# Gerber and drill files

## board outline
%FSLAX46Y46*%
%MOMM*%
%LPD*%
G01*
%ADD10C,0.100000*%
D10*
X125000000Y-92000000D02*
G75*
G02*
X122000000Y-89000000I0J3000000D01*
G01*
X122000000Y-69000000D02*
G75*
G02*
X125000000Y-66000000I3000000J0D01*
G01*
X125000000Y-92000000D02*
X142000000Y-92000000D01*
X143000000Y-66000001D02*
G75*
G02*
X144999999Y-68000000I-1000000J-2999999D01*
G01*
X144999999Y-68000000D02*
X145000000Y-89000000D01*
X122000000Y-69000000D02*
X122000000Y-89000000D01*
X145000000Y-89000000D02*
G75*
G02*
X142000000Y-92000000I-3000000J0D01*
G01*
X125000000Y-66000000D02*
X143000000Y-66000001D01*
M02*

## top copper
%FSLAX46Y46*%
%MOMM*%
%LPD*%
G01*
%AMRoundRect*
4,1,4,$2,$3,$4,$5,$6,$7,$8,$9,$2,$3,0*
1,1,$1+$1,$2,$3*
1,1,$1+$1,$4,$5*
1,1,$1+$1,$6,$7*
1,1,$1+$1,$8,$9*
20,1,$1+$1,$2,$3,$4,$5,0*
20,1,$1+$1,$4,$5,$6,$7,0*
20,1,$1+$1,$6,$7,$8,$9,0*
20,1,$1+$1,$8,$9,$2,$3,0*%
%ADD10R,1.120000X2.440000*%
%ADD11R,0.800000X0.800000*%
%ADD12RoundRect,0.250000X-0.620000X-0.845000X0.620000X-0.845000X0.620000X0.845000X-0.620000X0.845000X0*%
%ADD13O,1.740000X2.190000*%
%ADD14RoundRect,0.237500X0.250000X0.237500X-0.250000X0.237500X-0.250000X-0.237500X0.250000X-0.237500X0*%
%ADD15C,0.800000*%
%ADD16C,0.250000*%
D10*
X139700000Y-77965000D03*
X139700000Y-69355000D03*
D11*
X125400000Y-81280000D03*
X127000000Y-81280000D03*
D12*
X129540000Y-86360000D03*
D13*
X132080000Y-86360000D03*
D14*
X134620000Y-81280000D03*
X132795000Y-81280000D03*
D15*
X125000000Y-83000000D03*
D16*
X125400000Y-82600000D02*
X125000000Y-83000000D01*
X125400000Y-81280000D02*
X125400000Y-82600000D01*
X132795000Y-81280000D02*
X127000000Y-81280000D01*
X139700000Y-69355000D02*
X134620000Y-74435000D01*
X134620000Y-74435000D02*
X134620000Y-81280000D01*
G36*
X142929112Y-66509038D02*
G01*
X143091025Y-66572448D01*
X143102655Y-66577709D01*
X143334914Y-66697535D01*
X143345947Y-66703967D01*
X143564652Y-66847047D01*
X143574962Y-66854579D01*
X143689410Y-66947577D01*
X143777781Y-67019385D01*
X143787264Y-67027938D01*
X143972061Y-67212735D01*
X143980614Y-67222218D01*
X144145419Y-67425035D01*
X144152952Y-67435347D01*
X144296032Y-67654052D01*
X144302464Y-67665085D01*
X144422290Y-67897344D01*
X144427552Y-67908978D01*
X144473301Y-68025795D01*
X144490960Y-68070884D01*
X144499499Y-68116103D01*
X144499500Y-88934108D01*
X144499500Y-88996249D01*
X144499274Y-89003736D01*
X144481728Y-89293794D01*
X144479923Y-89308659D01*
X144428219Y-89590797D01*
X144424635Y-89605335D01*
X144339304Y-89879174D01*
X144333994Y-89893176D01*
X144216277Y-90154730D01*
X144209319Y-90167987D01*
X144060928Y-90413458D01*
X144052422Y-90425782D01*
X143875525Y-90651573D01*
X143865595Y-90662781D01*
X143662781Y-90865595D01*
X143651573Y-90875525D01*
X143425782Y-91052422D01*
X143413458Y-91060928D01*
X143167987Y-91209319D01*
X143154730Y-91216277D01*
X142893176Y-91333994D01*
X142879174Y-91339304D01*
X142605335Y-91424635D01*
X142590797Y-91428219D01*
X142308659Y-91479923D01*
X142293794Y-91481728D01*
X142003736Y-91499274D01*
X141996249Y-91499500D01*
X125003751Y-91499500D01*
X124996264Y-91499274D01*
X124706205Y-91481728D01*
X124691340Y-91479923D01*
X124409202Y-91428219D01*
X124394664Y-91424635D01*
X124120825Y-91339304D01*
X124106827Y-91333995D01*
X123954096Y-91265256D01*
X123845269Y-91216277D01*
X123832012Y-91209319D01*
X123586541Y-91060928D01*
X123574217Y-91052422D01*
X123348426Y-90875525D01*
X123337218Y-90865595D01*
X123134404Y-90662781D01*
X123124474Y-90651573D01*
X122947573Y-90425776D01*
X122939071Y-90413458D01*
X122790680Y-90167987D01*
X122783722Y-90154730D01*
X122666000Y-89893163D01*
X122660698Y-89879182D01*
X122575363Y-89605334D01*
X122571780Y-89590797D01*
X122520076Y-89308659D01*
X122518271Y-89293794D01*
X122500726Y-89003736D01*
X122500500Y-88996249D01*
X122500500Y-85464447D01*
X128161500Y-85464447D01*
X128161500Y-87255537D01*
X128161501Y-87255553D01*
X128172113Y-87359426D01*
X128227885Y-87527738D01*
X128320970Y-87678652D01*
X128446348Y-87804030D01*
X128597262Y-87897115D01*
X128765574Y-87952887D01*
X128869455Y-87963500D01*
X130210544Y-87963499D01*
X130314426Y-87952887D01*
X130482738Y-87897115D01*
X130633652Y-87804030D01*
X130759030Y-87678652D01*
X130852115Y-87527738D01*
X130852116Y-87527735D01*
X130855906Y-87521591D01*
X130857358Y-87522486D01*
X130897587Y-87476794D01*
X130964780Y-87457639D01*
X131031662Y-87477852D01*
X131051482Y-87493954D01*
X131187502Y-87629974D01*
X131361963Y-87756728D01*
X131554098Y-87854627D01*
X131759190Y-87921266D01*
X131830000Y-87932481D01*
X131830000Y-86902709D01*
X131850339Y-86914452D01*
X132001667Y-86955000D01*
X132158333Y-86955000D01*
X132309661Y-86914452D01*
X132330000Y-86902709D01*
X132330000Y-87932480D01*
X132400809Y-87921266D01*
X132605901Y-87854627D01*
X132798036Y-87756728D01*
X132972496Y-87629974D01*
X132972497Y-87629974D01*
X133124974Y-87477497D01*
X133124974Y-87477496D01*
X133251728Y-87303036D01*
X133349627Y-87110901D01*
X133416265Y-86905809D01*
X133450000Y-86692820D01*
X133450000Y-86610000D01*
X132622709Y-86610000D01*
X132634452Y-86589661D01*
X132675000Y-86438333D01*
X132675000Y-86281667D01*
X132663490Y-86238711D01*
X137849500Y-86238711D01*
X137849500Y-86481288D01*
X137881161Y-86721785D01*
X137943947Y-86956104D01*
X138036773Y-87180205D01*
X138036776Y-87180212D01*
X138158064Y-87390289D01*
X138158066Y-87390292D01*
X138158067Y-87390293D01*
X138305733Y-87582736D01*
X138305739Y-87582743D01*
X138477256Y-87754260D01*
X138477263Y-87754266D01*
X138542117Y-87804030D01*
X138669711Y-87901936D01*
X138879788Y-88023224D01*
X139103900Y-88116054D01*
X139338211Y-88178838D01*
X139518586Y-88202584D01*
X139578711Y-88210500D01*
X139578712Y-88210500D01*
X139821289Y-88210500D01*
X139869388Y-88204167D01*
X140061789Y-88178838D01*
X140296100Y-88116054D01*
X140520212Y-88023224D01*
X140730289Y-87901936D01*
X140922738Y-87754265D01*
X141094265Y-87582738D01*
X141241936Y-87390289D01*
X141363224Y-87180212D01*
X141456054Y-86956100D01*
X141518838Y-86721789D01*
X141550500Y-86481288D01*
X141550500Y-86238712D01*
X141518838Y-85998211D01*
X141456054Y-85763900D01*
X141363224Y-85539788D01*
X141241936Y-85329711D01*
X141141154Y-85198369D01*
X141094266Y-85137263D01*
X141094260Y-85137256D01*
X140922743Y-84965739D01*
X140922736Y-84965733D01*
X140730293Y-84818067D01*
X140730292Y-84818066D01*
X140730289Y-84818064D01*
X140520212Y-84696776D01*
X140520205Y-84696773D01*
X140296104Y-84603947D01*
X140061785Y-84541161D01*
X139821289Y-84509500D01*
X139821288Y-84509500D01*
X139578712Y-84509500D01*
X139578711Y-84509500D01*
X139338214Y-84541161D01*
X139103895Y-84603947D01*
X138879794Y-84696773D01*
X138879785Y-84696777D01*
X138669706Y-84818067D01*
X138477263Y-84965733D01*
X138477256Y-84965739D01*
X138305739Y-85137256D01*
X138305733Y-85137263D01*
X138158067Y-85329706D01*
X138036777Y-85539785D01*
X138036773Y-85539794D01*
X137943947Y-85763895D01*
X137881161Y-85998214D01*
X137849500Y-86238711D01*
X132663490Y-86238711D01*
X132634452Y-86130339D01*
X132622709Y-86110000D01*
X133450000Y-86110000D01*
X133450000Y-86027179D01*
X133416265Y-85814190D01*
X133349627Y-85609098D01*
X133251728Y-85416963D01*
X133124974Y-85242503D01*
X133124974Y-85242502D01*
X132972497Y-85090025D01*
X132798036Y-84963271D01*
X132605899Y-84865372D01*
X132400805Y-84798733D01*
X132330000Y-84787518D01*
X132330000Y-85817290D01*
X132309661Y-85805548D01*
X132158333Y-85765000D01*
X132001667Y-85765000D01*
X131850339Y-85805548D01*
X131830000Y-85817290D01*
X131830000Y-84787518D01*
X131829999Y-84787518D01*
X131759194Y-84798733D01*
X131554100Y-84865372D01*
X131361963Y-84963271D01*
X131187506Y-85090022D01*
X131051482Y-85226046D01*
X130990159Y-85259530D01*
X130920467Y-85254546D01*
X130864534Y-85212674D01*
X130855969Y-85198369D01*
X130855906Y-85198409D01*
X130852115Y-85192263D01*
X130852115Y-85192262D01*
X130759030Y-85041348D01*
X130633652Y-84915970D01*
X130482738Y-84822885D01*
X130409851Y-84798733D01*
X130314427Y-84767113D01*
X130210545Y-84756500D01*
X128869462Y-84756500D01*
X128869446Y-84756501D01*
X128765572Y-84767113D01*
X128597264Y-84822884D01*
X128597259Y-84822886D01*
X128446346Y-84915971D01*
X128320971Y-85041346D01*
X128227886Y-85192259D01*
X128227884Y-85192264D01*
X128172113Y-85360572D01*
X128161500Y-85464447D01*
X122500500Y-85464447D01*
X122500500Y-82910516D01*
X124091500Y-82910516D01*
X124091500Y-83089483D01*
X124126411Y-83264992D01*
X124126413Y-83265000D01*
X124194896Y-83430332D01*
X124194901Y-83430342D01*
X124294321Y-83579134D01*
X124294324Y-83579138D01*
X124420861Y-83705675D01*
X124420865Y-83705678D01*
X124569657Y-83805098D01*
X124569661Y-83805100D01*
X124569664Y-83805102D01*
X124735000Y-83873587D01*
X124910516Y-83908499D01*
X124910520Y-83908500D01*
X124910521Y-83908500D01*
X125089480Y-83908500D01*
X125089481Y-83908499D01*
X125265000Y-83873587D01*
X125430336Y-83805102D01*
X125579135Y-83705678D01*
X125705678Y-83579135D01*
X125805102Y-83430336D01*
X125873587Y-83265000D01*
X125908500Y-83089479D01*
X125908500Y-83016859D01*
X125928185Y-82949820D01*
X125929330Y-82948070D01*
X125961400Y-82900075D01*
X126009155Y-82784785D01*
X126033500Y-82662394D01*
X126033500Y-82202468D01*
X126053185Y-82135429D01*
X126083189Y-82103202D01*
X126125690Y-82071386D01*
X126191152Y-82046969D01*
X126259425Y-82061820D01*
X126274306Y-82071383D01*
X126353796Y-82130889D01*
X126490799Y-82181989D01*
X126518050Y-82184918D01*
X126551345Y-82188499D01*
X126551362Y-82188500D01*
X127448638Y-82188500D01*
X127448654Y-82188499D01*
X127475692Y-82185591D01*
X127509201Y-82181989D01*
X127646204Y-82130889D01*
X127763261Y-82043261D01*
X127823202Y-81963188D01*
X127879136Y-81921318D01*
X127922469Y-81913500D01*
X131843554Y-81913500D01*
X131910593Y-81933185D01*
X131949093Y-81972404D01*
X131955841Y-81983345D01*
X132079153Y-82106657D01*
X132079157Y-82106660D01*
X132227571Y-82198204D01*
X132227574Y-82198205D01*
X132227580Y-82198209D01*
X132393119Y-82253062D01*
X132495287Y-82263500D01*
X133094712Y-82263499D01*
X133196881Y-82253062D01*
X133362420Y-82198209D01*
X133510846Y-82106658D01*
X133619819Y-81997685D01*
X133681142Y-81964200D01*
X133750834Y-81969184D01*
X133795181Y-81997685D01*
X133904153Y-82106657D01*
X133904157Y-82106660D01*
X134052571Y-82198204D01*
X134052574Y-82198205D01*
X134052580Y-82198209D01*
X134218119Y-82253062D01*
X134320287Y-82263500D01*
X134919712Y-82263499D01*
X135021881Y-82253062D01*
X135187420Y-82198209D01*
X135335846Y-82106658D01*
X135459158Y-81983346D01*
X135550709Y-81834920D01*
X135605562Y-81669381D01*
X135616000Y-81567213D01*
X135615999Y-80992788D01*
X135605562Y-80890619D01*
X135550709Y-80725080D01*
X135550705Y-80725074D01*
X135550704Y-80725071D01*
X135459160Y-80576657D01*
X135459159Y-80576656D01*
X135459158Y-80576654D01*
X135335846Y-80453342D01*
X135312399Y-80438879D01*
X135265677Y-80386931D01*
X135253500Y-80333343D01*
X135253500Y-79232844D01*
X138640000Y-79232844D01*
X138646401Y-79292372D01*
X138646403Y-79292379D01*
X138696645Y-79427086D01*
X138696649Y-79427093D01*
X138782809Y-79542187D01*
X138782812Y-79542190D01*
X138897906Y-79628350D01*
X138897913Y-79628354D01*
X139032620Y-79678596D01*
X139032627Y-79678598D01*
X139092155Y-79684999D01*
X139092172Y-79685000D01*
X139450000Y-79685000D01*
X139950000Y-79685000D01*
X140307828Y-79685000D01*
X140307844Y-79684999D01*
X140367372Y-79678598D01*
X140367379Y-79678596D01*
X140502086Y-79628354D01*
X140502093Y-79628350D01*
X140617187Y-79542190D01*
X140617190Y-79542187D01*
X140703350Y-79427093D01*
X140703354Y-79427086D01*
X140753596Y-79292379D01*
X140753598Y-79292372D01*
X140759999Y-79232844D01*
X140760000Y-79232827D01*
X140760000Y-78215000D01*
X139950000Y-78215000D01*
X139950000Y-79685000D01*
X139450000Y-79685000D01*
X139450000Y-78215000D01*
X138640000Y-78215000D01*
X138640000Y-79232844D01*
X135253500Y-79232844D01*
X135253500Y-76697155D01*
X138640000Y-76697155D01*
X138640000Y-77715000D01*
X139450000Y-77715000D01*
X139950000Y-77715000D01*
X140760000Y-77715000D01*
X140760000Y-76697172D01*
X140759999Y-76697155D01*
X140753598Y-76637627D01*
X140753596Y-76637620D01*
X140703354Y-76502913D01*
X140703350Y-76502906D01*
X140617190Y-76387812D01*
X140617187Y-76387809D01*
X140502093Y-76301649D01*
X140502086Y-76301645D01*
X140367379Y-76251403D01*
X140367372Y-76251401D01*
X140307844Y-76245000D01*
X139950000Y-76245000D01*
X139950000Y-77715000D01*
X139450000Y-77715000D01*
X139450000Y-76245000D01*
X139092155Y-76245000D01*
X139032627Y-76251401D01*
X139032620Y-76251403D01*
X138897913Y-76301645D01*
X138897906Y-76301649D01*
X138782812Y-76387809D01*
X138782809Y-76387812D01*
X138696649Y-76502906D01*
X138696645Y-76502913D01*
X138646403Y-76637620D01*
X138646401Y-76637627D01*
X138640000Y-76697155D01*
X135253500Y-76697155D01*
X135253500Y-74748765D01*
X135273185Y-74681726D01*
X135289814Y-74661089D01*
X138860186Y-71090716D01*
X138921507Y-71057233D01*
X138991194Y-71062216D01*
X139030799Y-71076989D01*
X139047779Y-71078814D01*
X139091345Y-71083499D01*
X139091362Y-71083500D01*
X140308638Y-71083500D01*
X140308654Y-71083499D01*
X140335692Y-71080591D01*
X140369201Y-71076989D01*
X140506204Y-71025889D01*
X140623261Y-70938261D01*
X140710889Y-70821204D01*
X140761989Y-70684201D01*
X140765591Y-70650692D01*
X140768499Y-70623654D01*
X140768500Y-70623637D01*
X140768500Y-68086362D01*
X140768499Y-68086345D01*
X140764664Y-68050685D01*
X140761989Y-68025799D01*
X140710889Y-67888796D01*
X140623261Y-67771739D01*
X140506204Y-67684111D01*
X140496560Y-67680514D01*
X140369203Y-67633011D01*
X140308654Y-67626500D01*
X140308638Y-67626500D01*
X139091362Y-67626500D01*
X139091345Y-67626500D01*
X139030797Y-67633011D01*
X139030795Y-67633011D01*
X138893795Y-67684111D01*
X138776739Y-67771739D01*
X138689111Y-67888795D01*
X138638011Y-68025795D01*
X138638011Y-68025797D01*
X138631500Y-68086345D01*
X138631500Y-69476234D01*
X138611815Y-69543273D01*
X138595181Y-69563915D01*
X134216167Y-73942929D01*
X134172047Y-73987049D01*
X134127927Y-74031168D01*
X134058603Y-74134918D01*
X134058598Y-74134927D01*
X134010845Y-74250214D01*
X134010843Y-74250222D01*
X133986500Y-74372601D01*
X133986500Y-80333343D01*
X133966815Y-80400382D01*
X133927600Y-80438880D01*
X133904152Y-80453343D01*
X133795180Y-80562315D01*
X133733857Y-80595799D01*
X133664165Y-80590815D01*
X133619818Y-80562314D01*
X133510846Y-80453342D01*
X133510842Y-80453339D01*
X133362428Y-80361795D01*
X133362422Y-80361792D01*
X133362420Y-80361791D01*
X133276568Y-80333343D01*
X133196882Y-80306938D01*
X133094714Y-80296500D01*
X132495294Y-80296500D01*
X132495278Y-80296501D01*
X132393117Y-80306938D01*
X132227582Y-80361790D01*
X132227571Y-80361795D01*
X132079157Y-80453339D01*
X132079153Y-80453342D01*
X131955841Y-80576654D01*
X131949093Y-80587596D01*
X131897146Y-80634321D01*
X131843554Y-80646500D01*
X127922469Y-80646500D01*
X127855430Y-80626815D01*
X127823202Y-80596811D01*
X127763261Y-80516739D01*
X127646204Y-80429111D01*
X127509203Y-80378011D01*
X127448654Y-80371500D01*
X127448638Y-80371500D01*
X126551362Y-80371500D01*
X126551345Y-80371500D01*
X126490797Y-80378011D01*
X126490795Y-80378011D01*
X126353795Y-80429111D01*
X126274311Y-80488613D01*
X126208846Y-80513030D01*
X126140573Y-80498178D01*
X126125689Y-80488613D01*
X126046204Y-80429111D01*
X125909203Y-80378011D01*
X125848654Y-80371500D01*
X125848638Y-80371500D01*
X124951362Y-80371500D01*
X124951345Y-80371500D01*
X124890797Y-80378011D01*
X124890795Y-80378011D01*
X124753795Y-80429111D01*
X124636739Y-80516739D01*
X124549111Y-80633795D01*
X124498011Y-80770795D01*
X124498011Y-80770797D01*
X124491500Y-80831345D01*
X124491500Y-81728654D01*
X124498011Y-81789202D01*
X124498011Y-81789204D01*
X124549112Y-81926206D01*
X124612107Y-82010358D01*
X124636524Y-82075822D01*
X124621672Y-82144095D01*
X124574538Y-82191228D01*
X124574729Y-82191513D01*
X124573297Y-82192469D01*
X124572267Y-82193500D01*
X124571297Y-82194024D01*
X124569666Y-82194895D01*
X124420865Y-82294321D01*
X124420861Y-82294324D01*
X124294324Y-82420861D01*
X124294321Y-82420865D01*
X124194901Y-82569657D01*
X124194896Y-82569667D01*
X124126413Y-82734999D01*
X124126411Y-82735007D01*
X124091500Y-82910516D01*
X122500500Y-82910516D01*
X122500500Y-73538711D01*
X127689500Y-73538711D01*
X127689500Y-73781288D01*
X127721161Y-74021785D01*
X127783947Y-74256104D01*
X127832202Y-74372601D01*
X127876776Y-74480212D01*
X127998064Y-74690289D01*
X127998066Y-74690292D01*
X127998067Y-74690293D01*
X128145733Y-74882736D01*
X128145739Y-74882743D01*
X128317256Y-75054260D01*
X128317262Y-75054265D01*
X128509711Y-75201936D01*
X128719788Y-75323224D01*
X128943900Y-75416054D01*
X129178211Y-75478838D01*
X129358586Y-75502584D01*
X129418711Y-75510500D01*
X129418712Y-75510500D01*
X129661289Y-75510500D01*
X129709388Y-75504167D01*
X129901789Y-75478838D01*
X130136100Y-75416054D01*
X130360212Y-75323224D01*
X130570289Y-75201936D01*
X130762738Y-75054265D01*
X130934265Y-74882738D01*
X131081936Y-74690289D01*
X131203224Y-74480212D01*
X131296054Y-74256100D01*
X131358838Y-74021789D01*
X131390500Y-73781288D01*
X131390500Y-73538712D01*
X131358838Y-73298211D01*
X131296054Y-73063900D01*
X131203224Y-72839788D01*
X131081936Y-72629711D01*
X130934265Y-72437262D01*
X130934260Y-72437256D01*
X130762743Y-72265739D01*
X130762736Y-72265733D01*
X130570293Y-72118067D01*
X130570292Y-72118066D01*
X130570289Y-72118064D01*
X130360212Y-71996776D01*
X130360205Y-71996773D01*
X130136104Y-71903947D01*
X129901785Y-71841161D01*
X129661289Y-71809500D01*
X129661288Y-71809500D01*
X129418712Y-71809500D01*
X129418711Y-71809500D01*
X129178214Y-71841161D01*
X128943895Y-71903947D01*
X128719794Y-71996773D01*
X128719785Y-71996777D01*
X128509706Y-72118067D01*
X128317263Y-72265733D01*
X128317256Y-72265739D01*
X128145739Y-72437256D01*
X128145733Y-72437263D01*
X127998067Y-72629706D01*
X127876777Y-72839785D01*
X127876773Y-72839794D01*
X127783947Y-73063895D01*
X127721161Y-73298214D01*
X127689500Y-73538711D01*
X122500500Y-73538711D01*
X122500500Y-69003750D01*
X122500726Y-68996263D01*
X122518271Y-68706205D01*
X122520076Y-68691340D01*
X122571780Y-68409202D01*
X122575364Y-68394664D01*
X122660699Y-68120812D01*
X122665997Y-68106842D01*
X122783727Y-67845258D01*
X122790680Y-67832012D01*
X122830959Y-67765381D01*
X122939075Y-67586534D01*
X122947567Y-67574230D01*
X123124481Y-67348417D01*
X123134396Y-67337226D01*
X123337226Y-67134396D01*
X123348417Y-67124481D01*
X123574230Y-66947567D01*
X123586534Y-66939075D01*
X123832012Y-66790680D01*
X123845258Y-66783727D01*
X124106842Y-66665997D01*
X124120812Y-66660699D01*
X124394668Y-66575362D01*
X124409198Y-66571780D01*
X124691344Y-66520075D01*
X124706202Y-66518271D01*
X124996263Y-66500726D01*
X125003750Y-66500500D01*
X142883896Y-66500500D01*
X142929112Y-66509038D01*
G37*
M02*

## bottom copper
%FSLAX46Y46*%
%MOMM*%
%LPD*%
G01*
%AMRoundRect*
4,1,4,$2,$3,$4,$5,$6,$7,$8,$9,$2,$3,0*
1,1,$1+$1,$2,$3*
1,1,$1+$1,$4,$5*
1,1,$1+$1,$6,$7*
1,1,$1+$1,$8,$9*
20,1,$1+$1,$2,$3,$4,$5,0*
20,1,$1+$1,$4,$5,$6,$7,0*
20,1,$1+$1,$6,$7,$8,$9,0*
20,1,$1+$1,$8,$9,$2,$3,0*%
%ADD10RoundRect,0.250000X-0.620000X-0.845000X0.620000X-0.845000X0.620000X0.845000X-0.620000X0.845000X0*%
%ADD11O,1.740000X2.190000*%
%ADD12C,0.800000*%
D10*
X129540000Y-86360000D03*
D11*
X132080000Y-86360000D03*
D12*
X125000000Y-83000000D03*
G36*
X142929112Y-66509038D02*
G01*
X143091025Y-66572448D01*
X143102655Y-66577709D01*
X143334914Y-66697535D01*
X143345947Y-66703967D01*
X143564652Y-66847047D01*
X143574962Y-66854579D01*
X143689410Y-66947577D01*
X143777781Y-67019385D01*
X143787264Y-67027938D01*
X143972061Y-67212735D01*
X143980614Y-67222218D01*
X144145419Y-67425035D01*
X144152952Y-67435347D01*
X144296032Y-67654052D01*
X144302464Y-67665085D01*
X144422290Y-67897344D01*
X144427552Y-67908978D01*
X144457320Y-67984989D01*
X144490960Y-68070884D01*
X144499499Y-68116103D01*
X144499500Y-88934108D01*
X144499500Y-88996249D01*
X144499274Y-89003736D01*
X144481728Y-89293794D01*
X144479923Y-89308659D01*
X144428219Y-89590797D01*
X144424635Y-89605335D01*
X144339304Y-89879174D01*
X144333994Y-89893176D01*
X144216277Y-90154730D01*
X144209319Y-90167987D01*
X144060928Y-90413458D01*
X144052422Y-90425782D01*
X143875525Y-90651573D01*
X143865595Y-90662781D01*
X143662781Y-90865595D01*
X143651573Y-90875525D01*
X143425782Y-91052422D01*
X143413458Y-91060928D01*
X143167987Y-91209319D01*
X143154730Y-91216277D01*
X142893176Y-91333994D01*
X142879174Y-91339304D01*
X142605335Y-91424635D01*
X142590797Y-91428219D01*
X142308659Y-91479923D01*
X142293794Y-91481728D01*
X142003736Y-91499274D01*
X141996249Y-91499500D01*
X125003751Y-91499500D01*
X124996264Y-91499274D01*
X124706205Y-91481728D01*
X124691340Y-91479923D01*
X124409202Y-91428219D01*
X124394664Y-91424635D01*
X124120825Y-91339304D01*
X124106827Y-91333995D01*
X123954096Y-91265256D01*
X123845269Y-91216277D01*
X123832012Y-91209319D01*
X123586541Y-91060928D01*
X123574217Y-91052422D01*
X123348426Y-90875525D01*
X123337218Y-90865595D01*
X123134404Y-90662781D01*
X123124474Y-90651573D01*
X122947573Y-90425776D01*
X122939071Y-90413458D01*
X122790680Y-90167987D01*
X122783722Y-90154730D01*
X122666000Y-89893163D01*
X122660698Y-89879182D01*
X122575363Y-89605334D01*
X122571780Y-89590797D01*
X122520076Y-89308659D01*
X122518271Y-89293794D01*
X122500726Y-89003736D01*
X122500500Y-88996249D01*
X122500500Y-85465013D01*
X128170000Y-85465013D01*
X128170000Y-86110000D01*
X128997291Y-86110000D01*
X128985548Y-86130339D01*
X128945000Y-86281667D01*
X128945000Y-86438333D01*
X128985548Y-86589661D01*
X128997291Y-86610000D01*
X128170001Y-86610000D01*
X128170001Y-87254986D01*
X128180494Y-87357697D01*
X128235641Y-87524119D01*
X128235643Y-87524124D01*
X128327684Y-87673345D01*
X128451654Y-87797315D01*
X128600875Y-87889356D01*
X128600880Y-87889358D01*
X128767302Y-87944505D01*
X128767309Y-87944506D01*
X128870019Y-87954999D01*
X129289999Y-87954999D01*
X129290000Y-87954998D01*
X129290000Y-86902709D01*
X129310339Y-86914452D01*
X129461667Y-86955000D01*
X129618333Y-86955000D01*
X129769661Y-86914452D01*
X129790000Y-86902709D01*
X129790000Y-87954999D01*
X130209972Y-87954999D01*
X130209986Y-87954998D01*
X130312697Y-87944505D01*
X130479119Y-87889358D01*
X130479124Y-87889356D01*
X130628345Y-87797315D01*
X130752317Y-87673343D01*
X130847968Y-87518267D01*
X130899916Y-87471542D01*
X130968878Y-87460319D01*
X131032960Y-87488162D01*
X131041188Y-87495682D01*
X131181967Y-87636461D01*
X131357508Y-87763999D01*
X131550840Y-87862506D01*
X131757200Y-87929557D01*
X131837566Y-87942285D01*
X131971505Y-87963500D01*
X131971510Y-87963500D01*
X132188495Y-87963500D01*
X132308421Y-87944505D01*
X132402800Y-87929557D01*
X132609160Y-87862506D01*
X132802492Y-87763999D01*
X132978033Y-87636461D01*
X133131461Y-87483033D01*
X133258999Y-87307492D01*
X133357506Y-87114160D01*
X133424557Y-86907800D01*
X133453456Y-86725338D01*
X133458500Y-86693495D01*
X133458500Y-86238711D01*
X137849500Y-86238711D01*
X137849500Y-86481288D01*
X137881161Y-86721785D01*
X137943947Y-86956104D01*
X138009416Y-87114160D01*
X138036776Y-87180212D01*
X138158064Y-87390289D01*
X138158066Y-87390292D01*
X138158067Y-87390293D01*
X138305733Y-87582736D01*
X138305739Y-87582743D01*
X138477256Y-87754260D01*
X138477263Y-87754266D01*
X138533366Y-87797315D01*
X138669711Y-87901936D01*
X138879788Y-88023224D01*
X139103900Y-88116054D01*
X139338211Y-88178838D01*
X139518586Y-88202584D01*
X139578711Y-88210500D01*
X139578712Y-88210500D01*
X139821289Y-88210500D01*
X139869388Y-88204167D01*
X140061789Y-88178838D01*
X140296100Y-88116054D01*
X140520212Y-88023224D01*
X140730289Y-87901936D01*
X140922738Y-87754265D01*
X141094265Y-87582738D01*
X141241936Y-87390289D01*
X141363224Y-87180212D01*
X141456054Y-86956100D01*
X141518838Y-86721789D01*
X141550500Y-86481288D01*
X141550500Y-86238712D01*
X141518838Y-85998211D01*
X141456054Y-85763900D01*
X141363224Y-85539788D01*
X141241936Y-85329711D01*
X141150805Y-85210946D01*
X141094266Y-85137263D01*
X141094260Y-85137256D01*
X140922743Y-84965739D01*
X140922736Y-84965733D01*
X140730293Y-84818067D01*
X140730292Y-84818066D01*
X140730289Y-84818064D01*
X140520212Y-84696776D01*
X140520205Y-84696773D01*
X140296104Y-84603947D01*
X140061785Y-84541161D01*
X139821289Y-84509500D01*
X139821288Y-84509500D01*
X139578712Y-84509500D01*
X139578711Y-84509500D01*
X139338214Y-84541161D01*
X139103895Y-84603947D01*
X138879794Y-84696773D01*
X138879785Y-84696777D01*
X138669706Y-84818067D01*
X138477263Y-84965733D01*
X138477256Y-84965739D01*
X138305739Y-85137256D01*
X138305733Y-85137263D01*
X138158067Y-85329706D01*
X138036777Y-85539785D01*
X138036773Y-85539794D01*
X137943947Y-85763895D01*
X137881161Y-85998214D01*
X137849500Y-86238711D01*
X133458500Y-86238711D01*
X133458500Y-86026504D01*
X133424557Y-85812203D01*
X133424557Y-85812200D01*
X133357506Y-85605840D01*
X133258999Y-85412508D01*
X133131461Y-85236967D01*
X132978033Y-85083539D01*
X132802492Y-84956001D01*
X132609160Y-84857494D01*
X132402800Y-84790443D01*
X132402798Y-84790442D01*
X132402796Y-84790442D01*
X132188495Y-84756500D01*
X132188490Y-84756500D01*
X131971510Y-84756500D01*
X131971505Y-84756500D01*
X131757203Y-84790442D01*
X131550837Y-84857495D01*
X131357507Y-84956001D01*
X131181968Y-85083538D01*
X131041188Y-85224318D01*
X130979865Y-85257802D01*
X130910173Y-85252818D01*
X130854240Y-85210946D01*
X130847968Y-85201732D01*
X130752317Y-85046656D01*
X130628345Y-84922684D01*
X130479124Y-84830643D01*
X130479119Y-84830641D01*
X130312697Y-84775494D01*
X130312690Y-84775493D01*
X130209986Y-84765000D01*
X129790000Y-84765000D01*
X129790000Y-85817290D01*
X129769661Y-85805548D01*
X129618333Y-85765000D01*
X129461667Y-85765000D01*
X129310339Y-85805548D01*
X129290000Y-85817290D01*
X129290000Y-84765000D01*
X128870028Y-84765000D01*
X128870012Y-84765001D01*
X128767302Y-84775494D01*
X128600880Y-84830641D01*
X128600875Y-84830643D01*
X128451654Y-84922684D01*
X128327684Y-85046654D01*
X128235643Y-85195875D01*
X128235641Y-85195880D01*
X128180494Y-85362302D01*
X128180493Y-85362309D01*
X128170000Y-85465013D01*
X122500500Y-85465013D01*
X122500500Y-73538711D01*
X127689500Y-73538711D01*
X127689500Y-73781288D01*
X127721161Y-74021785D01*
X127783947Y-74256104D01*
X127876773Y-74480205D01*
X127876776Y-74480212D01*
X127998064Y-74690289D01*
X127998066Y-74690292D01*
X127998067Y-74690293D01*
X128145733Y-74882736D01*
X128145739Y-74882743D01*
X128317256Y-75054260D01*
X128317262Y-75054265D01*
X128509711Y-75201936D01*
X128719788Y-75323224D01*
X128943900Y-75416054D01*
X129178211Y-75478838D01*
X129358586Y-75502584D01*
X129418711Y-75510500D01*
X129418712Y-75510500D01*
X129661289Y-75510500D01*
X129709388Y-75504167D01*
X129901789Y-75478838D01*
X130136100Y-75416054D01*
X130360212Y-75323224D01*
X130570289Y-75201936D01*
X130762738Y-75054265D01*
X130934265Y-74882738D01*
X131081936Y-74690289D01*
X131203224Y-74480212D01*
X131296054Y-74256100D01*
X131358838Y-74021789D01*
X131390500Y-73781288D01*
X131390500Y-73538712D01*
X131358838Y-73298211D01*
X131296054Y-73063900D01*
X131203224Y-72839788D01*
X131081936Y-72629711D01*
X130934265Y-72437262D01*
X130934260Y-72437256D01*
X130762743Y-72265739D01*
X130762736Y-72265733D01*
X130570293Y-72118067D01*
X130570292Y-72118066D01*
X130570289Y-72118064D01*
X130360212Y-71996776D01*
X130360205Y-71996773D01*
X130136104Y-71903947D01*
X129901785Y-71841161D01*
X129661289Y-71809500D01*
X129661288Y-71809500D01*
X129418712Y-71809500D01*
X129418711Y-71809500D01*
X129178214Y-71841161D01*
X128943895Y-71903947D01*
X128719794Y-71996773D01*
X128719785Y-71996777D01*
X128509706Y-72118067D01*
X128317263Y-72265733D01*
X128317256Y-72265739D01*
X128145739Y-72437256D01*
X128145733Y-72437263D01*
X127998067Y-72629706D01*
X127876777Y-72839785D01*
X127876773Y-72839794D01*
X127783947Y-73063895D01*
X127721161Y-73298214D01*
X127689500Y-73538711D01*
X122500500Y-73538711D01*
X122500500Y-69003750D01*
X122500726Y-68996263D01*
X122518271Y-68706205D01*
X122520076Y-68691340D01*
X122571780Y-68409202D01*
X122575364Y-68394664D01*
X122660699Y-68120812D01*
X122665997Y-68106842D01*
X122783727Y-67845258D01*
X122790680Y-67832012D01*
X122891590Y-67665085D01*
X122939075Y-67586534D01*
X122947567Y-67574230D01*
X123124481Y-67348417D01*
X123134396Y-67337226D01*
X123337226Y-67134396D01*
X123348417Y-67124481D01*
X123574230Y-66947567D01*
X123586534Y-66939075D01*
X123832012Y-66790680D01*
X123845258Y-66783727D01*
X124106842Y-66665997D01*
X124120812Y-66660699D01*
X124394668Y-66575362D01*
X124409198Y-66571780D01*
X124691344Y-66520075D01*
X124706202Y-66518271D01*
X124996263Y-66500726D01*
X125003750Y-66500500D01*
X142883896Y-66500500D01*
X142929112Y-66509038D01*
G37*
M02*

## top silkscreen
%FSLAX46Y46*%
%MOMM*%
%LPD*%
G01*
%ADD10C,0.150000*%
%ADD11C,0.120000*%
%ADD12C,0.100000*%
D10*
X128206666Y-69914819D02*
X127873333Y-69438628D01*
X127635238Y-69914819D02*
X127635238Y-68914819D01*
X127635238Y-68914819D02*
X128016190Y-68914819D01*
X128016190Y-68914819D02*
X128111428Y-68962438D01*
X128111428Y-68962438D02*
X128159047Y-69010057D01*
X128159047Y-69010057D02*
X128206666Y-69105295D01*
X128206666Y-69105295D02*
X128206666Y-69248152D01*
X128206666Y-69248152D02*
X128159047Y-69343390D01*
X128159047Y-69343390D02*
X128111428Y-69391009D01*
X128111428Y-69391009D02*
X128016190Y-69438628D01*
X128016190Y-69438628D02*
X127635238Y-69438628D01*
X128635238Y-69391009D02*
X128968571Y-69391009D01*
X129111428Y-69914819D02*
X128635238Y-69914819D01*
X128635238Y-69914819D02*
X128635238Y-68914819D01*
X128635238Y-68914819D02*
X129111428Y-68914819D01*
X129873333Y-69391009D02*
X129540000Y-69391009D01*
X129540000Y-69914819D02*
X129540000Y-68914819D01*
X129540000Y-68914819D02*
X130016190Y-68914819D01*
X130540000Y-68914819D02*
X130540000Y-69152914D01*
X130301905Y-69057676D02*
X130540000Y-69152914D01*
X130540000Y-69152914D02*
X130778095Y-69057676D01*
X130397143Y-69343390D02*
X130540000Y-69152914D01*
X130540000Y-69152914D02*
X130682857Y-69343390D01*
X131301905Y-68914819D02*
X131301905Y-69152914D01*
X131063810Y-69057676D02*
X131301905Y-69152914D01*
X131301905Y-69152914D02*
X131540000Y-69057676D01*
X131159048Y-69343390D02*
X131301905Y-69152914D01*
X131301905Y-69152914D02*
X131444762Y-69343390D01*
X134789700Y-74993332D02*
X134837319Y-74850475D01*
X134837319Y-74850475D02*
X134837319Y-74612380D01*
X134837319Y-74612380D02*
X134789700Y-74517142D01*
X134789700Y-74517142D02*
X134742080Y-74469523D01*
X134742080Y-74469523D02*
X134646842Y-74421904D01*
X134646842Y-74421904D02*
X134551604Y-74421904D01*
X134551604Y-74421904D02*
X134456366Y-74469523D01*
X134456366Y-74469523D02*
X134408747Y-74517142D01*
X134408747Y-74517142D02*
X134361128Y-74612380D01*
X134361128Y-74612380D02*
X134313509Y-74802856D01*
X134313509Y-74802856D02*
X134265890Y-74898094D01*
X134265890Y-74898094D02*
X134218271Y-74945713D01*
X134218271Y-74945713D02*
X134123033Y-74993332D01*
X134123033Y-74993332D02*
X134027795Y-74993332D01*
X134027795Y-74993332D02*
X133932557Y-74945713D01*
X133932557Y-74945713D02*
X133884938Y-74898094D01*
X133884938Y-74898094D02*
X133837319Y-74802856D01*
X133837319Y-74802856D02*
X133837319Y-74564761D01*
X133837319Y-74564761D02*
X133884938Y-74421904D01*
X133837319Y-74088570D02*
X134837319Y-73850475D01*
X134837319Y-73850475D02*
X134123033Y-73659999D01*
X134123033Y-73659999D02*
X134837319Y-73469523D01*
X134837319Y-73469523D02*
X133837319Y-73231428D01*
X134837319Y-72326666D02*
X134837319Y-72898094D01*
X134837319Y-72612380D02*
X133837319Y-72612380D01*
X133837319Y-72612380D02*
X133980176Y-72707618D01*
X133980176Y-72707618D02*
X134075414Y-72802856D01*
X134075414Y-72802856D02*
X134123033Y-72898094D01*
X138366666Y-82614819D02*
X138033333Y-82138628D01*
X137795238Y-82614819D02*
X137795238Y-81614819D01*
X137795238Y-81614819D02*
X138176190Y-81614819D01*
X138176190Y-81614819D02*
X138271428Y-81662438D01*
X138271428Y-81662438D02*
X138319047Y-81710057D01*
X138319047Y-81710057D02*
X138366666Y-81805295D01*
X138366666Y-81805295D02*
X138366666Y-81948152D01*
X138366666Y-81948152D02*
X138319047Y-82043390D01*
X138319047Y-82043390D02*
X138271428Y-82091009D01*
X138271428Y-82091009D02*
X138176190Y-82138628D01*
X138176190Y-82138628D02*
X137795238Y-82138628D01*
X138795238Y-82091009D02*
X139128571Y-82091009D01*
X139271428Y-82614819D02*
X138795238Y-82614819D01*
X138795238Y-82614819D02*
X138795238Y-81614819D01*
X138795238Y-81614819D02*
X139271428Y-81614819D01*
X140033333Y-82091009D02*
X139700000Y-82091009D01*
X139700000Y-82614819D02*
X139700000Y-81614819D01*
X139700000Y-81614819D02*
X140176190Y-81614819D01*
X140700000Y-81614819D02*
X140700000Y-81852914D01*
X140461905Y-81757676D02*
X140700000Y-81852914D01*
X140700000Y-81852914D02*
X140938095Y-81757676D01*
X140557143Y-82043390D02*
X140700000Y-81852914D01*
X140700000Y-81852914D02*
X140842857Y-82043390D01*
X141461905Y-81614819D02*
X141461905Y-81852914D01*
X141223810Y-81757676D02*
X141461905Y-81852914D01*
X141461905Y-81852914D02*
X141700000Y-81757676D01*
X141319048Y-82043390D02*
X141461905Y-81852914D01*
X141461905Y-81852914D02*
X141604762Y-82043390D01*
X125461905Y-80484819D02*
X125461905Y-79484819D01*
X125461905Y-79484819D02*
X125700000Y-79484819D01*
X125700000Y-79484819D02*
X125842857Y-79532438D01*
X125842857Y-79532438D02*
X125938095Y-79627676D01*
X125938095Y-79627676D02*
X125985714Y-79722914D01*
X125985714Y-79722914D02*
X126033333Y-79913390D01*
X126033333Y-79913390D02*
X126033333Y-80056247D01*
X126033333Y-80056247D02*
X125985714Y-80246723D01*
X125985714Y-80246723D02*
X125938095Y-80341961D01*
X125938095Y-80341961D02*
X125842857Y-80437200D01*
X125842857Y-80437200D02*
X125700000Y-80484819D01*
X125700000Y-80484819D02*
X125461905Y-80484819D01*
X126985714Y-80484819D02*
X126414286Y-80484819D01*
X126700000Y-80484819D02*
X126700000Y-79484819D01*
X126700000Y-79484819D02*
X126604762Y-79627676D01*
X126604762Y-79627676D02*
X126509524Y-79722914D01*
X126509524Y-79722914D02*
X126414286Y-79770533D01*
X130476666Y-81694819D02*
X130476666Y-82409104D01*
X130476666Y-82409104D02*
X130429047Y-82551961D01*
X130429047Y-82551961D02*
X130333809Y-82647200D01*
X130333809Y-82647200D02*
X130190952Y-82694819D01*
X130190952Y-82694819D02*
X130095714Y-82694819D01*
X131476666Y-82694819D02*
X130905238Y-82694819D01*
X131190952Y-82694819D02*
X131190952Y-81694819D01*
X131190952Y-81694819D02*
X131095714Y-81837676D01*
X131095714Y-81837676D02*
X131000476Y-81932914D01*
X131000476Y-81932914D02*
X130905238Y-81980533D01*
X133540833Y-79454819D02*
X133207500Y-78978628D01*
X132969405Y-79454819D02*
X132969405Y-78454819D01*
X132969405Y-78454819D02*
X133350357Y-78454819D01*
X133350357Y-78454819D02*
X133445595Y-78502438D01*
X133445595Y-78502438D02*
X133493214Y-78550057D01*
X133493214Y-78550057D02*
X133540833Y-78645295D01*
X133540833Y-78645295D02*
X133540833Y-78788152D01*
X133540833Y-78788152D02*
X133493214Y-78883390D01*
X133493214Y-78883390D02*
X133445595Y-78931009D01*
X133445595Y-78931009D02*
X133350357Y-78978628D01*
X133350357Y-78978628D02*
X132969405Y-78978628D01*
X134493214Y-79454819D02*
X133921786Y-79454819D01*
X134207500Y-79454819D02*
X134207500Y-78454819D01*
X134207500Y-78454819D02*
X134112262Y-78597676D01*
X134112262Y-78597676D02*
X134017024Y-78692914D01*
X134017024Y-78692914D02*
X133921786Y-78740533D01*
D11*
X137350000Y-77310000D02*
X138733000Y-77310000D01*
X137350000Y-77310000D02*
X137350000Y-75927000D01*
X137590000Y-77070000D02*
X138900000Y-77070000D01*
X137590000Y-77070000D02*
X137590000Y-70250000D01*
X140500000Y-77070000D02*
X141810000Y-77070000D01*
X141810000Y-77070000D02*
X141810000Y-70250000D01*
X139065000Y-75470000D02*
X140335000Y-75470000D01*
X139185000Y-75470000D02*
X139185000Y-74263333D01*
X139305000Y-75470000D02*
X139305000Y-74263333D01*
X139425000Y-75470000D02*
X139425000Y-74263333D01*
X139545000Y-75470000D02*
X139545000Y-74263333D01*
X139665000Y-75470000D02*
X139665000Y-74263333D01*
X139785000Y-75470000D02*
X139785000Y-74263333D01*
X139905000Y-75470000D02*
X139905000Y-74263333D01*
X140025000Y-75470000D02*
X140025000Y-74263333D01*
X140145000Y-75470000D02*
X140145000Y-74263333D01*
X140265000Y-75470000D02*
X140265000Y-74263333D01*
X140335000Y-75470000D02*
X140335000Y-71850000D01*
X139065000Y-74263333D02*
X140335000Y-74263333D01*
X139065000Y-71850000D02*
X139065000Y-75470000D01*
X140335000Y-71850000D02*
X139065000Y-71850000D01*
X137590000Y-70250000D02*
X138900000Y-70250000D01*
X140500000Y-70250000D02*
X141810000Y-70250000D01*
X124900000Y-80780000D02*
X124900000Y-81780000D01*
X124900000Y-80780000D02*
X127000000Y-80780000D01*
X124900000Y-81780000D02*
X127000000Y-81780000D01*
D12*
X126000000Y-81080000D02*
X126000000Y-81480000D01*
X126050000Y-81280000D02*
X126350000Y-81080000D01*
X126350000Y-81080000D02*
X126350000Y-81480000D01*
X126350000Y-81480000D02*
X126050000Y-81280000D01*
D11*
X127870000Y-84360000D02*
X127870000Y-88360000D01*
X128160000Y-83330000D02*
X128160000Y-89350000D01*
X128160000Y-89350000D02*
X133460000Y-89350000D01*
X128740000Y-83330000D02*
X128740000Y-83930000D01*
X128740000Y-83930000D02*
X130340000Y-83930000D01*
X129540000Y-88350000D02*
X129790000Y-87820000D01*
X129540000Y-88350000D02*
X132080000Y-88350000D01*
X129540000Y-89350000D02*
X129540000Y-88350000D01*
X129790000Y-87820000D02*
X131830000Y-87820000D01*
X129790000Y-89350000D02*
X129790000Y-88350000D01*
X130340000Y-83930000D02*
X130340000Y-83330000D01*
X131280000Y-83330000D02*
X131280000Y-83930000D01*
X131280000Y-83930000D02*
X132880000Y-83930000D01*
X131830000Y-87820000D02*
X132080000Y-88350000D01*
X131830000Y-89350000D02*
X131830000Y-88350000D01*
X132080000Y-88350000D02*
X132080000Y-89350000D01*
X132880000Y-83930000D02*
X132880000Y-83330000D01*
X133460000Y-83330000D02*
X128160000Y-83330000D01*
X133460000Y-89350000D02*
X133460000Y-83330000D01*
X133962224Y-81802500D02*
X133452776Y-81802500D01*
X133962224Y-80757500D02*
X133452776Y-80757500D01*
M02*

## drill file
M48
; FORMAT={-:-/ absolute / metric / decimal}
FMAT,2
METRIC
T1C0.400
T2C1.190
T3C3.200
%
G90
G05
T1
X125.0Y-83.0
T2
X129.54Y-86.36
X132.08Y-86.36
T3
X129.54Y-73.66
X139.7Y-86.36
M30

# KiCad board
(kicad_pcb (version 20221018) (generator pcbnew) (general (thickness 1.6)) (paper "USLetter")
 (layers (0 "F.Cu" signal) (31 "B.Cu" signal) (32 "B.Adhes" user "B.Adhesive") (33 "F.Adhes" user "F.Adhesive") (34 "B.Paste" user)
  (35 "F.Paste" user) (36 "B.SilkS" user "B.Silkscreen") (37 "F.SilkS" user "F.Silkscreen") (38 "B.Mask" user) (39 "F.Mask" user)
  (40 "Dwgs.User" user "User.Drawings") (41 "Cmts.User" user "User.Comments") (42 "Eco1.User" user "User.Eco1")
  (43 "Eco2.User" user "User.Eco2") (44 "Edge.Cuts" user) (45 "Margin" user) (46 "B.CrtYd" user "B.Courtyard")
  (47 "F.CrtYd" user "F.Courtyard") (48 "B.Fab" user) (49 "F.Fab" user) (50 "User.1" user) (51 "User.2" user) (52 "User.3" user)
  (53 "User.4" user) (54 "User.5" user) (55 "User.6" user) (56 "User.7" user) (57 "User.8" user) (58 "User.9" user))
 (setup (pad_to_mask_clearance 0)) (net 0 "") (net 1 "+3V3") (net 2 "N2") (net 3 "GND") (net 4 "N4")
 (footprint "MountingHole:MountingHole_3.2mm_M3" (layer "F.Cu") (at 129.54 73.66)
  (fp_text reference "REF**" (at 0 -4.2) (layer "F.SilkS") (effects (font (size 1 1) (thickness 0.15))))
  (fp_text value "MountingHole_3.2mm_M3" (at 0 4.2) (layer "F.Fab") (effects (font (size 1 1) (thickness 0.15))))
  (pad "" np_thru_hole circle (at 0 0) (size 3.2 3.2) (drill 3.2) (layers "*.Cu" "*.Mask")))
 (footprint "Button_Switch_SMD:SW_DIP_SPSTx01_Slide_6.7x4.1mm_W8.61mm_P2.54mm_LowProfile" (layer "F.Cu") (at 139.7 73.66 90)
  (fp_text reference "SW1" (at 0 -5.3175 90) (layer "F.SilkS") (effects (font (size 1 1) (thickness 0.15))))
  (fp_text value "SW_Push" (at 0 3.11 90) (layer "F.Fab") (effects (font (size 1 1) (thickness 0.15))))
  (fp_line (start -3.65 -2.35) (end -3.65 -0.967) (stroke (width 0.12) (type solid)) (layer "F.SilkS"))
  (fp_line (start -3.65 -2.35) (end -2.267 -2.35) (stroke (width 0.12) (type solid)) (layer "F.SilkS"))
  (fp_line (start -3.41 -2.11) (end -3.41 -0.8) (stroke (width 0.12) (type solid)) (layer "F.SilkS"))
  (fp_line (start -3.41 -2.11) (end 3.41 -2.11) (stroke (width 0.12) (type solid)) (layer "F.SilkS"))
  (fp_line (start -3.41 0.8) (end -3.41 2.11) (stroke (width 0.12) (type solid)) (layer "F.SilkS"))
  (fp_line (start -3.41 2.11) (end 3.41 2.11) (stroke (width 0.12) (type solid)) (layer "F.SilkS"))
  (fp_line (start -1.81 -0.635) (end -1.81 0.635) (stroke (width 0.12) (type solid)) (layer "F.SilkS"))
  (fp_line (start -1.81 -0.515) (end -0.603333 -0.515) (stroke (width 0.12) (type solid)) (layer "F.SilkS"))
  (fp_line (start -1.81 -0.395) (end -0.603333 -0.395) (stroke (width 0.12) (type solid)) (layer "F.SilkS"))
  (fp_line (start -1.81 -0.275) (end -0.603333 -0.275) (stroke (width 0.12) (type solid)) (layer "F.SilkS"))
  (fp_line (start -1.81 -0.155) (end -0.603333 -0.155) (stroke (width 0.12) (type solid)) (layer "F.SilkS"))
  (fp_line (start -1.81 -0.035) (end -0.603333 -0.035) (stroke (width 0.12) (type solid)) (layer "F.SilkS"))
  (fp_line (start -1.81 0.085) (end -0.603333 0.085) (stroke (width 0.12) (type solid)) (layer "F.SilkS"))
  (fp_line (start -1.81 0.205) (end -0.603333 0.205) (stroke (width 0.12) (type solid)) (layer "F.SilkS"))
  (fp_line (start -1.81 0.325) (end -0.603333 0.325) (stroke (width 0.12) (type solid)) (layer "F.SilkS"))
  (fp_line (start -1.81 0.445) (end -0.603333 0.445) (stroke (width 0.12) (type solid)) (layer "F.SilkS"))
  (fp_line (start -1.81 0.565) (end -0.603333 0.565) (stroke (width 0.12) (type solid)) (layer "F.SilkS"))
  (fp_line (start -1.81 0.635) (end 1.81 0.635) (stroke (width 0.12) (type solid)) (layer "F.SilkS"))
  (fp_line (start -0.603333 -0.635) (end -0.603333 0.635) (stroke (width 0.12) (type solid)) (layer "F.SilkS"))
  (fp_line (start 1.81 -0.635) (end -1.81 -0.635) (stroke (width 0.12) (type solid)) (layer "F.SilkS"))
  (fp_line (start 1.81 0.635) (end 1.81 -0.635) (stroke (width 0.12) (type solid)) (layer "F.SilkS"))
  (fp_line (start 3.41 -2.11) (end 3.41 -0.8) (stroke (width 0.12) (type solid)) (layer "F.SilkS"))
  (fp_line (start 3.41 0.8) (end 3.41 2.11) (stroke (width 0.12) (type solid)) (layer "F.SilkS"))
  (pad "1" smd rect (at -4.305 0 90) (size 2.44 1.12) (layers "F.Cu" "F.Paste" "F.Mask") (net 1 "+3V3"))
  (pad "2" smd rect (at 4.305 0 90) (size 2.44 1.12) (layers "F.Cu" "F.Paste" "F.Mask") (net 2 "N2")))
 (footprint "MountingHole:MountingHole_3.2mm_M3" (layer "F.Cu") (at 139.7 86.36)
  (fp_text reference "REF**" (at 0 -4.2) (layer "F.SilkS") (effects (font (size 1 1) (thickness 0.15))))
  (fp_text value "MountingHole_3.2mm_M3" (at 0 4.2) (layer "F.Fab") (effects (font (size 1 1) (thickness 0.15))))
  (pad "" np_thru_hole circle (at 0 0) (size 3.2 3.2) (drill 3.2) (layers "*.Cu" "*.Mask")))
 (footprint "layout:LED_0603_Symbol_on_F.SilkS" (layer "F.Cu") (at 126.2 81.28)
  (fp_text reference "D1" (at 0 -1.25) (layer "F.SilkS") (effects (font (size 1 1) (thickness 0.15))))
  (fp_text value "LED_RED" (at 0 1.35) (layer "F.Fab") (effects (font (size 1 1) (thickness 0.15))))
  (fp_line (start -1.3 -0.5) (end -1.3 0.5) (stroke (width 0.12) (type solid)) (layer "F.SilkS"))
  (fp_line (start -1.3 -0.5) (end 0.8 -0.5) (stroke (width 0.12) (type solid)) (layer "F.SilkS"))
  (fp_line (start -1.3 0.5) (end 0.8 0.5) (stroke (width 0.12) (type solid)) (layer "F.SilkS"))
  (fp_line (start -0.2 -0.2) (end -0.2 0.2) (stroke (width 0.1) (type solid)) (layer "F.SilkS"))
  (fp_line (start -0.15 0) (end 0.15 -0.2) (stroke (width 0.1) (type solid)) (layer "F.SilkS"))
  (fp_line (start 0.15 -0.2) (end 0.15 0.2) (stroke (width 0.1) (type solid)) (layer "F.SilkS"))
  (fp_line (start 0.15 0.2) (end -0.15 0) (stroke (width 0.1) (type solid)) (layer "F.SilkS"))
  (pad "1" smd rect (at -0.8 0 180) (size 0.8 0.8) (layers "F.Cu" "F.Paste" "F.Mask") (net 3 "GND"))
  (pad "2" smd rect (at 0.8 0 180) (size 0.8 0.8) (layers "F.Cu" "F.Paste" "F.Mask") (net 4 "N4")))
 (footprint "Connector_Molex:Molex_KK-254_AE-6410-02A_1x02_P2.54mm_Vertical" (layer "F.Cu") (at 129.54 86.36)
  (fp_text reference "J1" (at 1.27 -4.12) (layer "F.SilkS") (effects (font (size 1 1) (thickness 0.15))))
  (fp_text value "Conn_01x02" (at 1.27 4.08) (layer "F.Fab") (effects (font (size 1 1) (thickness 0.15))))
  (fp_line (start -1.67 -2) (end -1.67 2) (stroke (width 0.12) (type solid)) (layer "F.SilkS"))
  (fp_line (start -1.38 -3.03) (end -1.38 2.99) (stroke (width 0.12) (type solid)) (layer "F.SilkS"))
  (fp_line (start -1.38 2.99) (end 3.92 2.99) (stroke (width 0.12) (type solid)) (layer "F.SilkS"))
  (fp_line (start -0.8 -3.03) (end -0.8 -2.43) (stroke (width 0.12) (type solid)) (layer "F.SilkS"))
  (fp_line (start -0.8 -2.43) (end 0.8 -2.43) (stroke (width 0.12) (type solid)) (layer "F.SilkS"))
  (fp_line (start 0 1.99) (end 0.25 1.46) (stroke (width 0.12) (type solid)) (layer "F.SilkS"))
  (fp_line (start 0 1.99) (end 2.54 1.99) (stroke (width 0.12) (type solid)) (layer "F.SilkS"))
  (fp_line (start 0 2.99) (end 0 1.99) (stroke (width 0.12) (type solid)) (layer "F.SilkS"))
  (fp_line (start 0.25 1.46) (end 2.29 1.46) (stroke (width 0.12) (type solid)) (layer "F.SilkS"))
  (fp_line (start 0.25 2.99) (end 0.25 1.99) (stroke (width 0.12) (type solid)) (layer "F.SilkS"))
  (fp_line (start 0.8 -2.43) (end 0.8 -3.03) (stroke (width 0.12) (type solid)) (layer "F.SilkS"))
  (fp_line (start 1.74 -3.03) (end 1.74 -2.43) (stroke (width 0.12) (type solid)) (layer "F.SilkS"))
  (fp_line (start 1.74 -2.43) (end 3.34 -2.43) (stroke (width 0.12) (type solid)) (layer "F.SilkS"))
  (fp_line (start 2.29 1.46) (end 2.54 1.99) (stroke (width 0.12) (type solid)) (layer "F.SilkS"))
  (fp_line (start 2.29 2.99) (end 2.29 1.99) (stroke (width 0.12) (type solid)) (layer "F.SilkS"))
  (fp_line (start 2.54 1.99) (end 2.54 2.99) (stroke (width 0.12) (type solid)) (layer "F.SilkS"))
  (fp_line (start 3.34 -2.43) (end 3.34 -3.03) (stroke (width 0.12) (type solid)) (layer "F.SilkS"))
  (fp_line (start 3.92 -3.03) (end -1.38 -3.03) (stroke (width 0.12) (type solid)) (layer "F.SilkS"))
  (fp_line (start 3.92 2.99) (end 3.92 -3.03) (stroke (width 0.12) (type solid)) (layer "F.SilkS"))
  (pad "1" thru_hole roundrect (at 0 0) (size 1.74 2.19) (drill 1.19) (layers "*.Cu" "*.Mask") (roundrect_rratio 0.143678) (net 3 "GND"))
  (pad "2" thru_hole oval (at 2.54 0) (size 1.74 2.19) (drill 1.19) (layers "*.Cu" "*.Mask") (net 1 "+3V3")))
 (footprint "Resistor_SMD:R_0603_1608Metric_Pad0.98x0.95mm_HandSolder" (layer "F.Cu") (at 133.7075 81.28 180)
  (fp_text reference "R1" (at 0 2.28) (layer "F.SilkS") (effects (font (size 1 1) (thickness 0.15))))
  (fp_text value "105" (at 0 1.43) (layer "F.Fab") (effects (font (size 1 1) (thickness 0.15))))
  (fp_line (start -0.254724 -0.5225) (end 0.254724 -0.5225) (stroke (width 0.12) (type solid)) (layer "F.SilkS"))
  (fp_line (start -0.254724 0.5225) (end 0.254724 0.5225) (stroke (width 0.12) (type solid)) (layer "F.SilkS"))
  (pad "1" smd roundrect (at -0.9125 0 180) (size 0.975 0.95) (layers "F.Cu" "F.Paste" "F.Mask") (roundrect_rratio 0.25) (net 2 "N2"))
  (pad "2" smd roundrect (at 0.9125 0 180) (size 0.975 0.95) (layers "F.Cu" "F.Paste" "F.Mask") (roundrect_rratio 0.25) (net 4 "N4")))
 (gr_arc (start 125 92) (mid 122.87868 91.12132) (end 122 89) (stroke (width 0.1) (type default)) (layer "Edge.Cuts"))
 (gr_arc (start 122 69) (mid 122.87868 66.87868) (end 125 66) (stroke (width 0.1) (type default)) (layer "Edge.Cuts"))
 (gr_line (start 125 92) (end 142 92) (stroke (width 0.1) (type default)) (layer "Edge.Cuts"))
 (gr_arc (start 143 66.000001) (mid 144.236067 66.763933) (end 144.999999 68) (stroke (width 0.1) (type default)) (layer "Edge.Cuts"))
 (gr_line (start 144.999999 68) (end 145 89) (stroke (width 0.1) (type default)) (layer "Edge.Cuts"))
 (gr_line (start 122 69) (end 122 89) (stroke (width 0.1) (type default)) (layer "Edge.Cuts"))
 (gr_arc (start 145 89) (mid 144.12132 91.12132) (end 142 92) (stroke (width 0.1) (type default)) (layer "Edge.Cuts"))
 (gr_line (start 125 66) (end 143 66.000001) (stroke (width 0.1) (type default)) (layer "Edge.Cuts"))
 (segment (start 125.4 82.6) (end 125 83) (width 0.25) (layer "F.Cu") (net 3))
 (segment (start 125.4 81.28) (end 125.4 82.6) (width 0.25) (layer "F.Cu") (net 3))
 (via (at 125 83) (size 0.8) (drill 0.4) (layers "F.Cu" "B.Cu") (free) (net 3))
 (segment (start 132.795 81.28) (end 127 81.28) (width 0.25) (layer "F.Cu") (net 4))
 (segment (start 139.7 69.355) (end 134.62 74.435) (width 0.25) (layer "F.Cu") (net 2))
 (segment (start 134.62 74.435) (end 134.62 81.28) (width 0.25) (layer "F.Cu") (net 2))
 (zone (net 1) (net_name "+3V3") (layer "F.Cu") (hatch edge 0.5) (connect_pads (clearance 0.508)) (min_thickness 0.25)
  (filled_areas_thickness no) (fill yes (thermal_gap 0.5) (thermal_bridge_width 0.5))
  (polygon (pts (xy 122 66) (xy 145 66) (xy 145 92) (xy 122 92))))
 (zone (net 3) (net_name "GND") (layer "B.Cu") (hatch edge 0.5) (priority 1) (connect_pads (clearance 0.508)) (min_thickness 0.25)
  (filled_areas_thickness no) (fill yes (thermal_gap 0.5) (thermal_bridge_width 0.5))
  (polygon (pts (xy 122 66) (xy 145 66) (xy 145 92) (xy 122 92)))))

